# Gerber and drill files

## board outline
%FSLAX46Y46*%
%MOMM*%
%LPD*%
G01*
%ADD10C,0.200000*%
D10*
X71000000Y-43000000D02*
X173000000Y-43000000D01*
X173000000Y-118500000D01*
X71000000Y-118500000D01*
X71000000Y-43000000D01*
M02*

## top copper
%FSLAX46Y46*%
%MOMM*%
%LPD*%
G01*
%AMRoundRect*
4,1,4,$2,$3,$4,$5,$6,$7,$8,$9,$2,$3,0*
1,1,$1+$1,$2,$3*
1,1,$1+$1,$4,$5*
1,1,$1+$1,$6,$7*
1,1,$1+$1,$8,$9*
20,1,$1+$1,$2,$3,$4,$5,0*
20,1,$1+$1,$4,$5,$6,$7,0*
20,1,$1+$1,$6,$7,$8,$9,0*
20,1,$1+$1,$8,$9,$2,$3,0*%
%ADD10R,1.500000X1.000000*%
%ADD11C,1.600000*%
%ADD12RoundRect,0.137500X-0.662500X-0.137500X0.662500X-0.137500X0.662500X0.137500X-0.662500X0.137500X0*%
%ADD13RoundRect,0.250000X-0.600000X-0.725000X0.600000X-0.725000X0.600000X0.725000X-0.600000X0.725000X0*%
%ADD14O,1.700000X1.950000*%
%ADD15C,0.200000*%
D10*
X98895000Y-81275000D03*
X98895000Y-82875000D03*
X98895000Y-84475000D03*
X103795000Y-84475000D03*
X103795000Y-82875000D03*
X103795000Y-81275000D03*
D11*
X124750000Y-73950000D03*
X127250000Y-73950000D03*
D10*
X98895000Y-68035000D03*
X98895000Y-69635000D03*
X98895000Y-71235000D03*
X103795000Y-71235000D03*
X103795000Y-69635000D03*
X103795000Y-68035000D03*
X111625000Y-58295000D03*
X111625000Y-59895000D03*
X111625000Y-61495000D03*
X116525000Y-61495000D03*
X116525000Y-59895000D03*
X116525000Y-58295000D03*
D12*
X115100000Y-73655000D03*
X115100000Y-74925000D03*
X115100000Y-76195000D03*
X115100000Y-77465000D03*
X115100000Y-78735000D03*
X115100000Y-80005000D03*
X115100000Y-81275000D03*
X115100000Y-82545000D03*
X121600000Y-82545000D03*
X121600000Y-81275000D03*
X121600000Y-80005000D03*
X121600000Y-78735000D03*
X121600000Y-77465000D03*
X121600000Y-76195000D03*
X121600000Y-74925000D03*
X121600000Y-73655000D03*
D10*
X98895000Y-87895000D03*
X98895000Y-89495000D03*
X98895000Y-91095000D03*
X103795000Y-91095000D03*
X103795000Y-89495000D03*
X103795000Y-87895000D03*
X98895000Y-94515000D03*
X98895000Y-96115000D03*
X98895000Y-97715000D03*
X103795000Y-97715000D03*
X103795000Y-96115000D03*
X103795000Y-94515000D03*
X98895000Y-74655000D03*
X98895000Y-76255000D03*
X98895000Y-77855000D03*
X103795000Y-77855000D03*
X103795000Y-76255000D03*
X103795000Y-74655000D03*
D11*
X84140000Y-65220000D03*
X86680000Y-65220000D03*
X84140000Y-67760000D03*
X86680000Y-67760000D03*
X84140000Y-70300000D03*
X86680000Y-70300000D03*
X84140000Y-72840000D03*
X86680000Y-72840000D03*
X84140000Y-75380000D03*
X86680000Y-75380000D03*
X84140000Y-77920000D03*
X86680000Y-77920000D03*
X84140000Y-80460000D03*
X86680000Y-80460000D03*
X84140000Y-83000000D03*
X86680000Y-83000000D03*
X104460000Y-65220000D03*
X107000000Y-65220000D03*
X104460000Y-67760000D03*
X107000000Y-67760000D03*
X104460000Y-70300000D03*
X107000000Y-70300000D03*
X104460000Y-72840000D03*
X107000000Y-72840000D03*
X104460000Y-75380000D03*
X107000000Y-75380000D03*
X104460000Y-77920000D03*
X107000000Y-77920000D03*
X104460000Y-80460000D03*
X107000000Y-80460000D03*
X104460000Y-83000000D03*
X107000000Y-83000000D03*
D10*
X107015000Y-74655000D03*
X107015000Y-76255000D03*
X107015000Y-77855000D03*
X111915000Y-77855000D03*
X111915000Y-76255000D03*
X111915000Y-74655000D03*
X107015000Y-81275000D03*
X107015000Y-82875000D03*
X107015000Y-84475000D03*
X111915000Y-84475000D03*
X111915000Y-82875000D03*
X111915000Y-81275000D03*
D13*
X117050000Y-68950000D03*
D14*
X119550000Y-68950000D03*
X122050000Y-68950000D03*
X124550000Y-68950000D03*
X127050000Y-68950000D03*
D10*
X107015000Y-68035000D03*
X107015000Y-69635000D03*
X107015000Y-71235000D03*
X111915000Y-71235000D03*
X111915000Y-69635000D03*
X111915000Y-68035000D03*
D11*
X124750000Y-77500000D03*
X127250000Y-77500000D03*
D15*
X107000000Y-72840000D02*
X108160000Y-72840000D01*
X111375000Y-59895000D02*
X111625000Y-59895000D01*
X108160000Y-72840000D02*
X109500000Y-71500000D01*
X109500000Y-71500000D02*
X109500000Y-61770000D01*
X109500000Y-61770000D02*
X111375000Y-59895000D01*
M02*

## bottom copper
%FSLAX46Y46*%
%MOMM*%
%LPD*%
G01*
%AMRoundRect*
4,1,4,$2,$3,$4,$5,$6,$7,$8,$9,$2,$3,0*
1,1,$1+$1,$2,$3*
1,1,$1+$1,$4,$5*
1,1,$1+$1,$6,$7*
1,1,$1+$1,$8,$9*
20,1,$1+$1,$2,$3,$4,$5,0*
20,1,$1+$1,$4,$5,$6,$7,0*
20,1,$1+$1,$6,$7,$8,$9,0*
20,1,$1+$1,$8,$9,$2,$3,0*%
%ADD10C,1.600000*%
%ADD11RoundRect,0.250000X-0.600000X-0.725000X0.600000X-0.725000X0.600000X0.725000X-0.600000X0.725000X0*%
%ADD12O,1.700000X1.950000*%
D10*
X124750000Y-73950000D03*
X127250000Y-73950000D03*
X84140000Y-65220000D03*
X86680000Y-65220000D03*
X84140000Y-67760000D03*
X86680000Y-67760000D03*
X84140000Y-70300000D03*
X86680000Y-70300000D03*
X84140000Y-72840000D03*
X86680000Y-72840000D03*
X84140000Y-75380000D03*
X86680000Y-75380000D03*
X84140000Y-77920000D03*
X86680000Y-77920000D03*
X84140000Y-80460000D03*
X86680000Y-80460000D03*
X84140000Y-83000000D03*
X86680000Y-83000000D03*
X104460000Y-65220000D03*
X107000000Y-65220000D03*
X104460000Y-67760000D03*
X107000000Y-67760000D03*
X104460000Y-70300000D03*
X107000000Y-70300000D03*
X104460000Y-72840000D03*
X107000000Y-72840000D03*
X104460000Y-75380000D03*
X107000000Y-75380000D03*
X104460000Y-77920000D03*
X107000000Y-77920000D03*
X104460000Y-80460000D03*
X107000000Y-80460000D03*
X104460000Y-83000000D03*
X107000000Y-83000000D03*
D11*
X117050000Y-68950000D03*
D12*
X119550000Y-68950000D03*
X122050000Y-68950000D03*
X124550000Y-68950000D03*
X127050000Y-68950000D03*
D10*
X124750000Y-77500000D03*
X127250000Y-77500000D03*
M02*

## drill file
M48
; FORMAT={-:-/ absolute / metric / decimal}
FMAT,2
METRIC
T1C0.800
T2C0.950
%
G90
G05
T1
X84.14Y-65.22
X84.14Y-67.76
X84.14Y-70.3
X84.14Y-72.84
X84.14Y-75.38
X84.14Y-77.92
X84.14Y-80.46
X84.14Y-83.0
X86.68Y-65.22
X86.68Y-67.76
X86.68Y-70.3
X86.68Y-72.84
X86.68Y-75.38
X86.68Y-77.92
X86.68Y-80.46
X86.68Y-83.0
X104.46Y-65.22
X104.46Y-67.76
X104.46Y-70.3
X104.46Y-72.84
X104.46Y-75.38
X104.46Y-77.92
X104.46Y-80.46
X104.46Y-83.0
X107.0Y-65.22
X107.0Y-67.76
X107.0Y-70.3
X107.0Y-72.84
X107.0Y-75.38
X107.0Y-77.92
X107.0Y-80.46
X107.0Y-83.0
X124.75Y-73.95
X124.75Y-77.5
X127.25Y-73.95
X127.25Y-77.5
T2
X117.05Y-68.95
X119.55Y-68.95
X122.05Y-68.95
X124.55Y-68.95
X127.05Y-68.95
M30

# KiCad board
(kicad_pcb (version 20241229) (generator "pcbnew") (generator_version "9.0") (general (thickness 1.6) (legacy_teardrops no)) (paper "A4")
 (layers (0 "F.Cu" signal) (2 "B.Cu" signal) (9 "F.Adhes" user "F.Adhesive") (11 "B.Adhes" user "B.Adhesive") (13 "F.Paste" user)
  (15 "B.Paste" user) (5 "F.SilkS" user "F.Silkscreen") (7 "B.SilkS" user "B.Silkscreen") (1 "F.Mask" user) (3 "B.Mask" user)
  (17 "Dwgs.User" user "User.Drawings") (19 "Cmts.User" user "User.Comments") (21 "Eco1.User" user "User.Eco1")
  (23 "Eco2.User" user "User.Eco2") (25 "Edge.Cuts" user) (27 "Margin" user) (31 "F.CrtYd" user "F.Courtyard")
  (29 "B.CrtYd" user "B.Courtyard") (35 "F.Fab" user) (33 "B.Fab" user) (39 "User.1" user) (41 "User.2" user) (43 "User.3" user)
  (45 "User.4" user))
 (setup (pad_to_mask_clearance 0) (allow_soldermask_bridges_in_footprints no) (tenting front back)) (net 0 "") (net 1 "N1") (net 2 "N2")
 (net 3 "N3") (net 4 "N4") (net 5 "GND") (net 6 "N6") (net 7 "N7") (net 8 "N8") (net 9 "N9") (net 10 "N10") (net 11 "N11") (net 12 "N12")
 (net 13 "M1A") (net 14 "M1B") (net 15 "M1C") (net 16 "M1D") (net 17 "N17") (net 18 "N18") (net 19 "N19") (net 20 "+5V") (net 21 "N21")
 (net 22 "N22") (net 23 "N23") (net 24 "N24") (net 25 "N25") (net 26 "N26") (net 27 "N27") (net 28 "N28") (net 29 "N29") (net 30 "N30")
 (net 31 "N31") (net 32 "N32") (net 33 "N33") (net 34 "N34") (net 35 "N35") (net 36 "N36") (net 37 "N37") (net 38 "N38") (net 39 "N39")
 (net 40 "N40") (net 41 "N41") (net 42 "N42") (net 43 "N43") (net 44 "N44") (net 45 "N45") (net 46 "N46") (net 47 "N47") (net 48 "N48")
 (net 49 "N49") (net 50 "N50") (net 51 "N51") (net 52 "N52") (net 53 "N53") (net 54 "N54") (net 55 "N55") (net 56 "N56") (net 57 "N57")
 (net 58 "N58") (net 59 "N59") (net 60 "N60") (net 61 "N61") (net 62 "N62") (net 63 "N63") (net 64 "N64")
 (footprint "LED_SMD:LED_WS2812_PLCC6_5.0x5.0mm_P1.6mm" (layer "F.Cu") (at 101.345 82.875)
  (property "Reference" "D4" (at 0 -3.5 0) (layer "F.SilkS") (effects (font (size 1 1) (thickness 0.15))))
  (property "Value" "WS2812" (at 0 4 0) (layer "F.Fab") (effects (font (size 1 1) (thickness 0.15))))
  (pad "1" smd rect (at -2.45 -1.6) (size 1.5 1) (layers "F.Cu" "F.Mask" "F.Paste") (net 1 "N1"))
  (pad "2" smd rect (at -2.45 0) (size 1.5 1) (layers "F.Cu" "F.Mask" "F.Paste") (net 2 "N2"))
  (pad "3" smd rect (at -2.45 1.6) (size 1.5 1) (layers "F.Cu" "F.Mask" "F.Paste") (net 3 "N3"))
  (pad "4" smd rect (at 2.45 1.6) (size 1.5 1) (layers "F.Cu" "F.Mask" "F.Paste") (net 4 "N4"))
  (pad "5" smd rect (at 2.45 0) (size 1.5 1) (layers "F.Cu" "F.Mask" "F.Paste") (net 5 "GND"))
  (pad "6" smd rect (at 2.45 -1.6) (size 1.5 1) (layers "F.Cu" "F.Mask" "F.Paste") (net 5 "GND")))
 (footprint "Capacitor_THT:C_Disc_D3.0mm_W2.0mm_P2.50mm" (layer "F.Cu") (at 124.75 73.95)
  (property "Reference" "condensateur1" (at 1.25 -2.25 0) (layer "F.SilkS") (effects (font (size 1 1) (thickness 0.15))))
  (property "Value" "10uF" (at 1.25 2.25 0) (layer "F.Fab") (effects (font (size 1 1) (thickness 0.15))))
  (pad "1" thru_hole circle (at 0 0) (size 1.6 1.6) (drill 0.8) (layers "*.Cu" "*.Mask") (remove_unused_layers no) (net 5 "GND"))
  (pad "2" thru_hole circle (at 2.5 0) (size 1.6 1.6) (drill 0.8) (layers "*.Cu" "*.Mask") (remove_unused_layers no) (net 5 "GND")))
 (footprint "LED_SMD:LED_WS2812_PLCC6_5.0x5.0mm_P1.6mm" (layer "F.Cu") (at 101.345 69.635)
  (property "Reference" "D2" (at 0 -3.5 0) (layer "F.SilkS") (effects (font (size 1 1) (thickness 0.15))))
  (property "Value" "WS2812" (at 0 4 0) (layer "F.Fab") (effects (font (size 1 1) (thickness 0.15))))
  (pad "1" smd rect (at -2.45 -1.6) (size 1.5 1) (layers "F.Cu" "F.Mask" "F.Paste") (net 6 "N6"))
  (pad "2" smd rect (at -2.45 0) (size 1.5 1) (layers "F.Cu" "F.Mask" "F.Paste") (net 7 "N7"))
  (pad "3" smd rect (at -2.45 1.6) (size 1.5 1) (layers "F.Cu" "F.Mask" "F.Paste") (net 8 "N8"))
  (pad "4" smd rect (at 2.45 1.6) (size 1.5 1) (layers "F.Cu" "F.Mask" "F.Paste") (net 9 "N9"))
  (pad "5" smd rect (at 2.45 0) (size 1.5 1) (layers "F.Cu" "F.Mask" "F.Paste") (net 5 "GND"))
  (pad "6" smd rect (at 2.45 -1.6) (size 1.5 1) (layers "F.Cu" "F.Mask" "F.Paste") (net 5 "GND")))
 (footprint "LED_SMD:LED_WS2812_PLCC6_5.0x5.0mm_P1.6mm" (layer "F.Cu") (at 114.075 59.895)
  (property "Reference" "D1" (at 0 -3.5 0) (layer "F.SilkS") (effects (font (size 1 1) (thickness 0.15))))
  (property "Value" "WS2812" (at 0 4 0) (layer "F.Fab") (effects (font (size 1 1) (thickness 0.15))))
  (pad "1" smd rect (at -2.45 -1.6) (size 1.5 1) (layers "F.Cu" "F.Mask" "F.Paste") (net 7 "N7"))
  (pad "2" smd rect (at -2.45 0) (size 1.5 1) (layers "F.Cu" "F.Mask" "F.Paste") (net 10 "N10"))
  (pad "3" smd rect (at -2.45 1.6) (size 1.5 1) (layers "F.Cu" "F.Mask" "F.Paste") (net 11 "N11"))
  (pad "4" smd rect (at 2.45 1.6) (size 1.5 1) (layers "F.Cu" "F.Mask" "F.Paste") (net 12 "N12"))
  (pad "5" smd rect (at 2.45 0) (size 1.5 1) (layers "F.Cu" "F.Mask" "F.Paste") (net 5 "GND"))
  (pad "6" smd rect (at 2.45 -1.6) (size 1.5 1) (layers "F.Cu" "F.Mask" "F.Paste") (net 5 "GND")))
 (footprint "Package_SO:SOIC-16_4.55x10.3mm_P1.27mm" (layer "F.Cu") (at 118.35 78.1)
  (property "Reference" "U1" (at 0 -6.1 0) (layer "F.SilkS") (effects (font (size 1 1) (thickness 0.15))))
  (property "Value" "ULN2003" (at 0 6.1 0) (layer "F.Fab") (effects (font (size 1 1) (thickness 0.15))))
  (pad "1" smd roundrect (at -3.25 -4.445) (size 1.6 0.55) (layers "F.Cu" "F.Mask" "F.Paste") (roundrect_rratio 0.25) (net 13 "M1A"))
  (pad "2" smd roundrect (at -3.25 -3.175) (size 1.6 0.55) (layers "F.Cu" "F.Mask" "F.Paste") (roundrect_rratio 0.25) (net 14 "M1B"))
  (pad "3" smd roundrect (at -3.25 -1.905) (size 1.6 0.55) (layers "F.Cu" "F.Mask" "F.Paste") (roundrect_rratio 0.25) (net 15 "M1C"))
  (pad "4" smd roundrect (at -3.25 -0.635) (size 1.6 0.55) (layers "F.Cu" "F.Mask" "F.Paste") (roundrect_rratio 0.25) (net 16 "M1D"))
  (pad "5" smd roundrect (at -3.25 0.635) (size 1.6 0.55) (layers "F.Cu" "F.Mask" "F.Paste") (roundrect_rratio 0.25) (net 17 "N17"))
  (pad "6" smd roundrect (at -3.25 1.905) (size 1.6 0.55) (layers "F.Cu" "F.Mask" "F.Paste") (roundrect_rratio 0.25) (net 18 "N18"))
  (pad "7" smd roundrect (at -3.25 3.175) (size 1.6 0.55) (layers "F.Cu" "F.Mask" "F.Paste") (roundrect_rratio 0.25) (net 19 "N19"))
  (pad "8" smd roundrect (at -3.25 4.445) (size 1.6 0.55) (layers "F.Cu" "F.Mask" "F.Paste") (roundrect_rratio 0.25) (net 5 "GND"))
  (pad "9" smd roundrect (at 3.25 4.445) (size 1.6 0.55) (layers "F.Cu" "F.Mask" "F.Paste") (roundrect_rratio 0.25) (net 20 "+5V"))
  (pad "10" smd roundrect (at 3.25 3.175) (size 1.6 0.55) (layers "F.Cu" "F.Mask" "F.Paste") (roundrect_rratio 0.25) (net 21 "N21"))
  (pad "11" smd roundrect (at 3.25 1.905) (size 1.6 0.55) (layers "F.Cu" "F.Mask" "F.Paste") (roundrect_rratio 0.25) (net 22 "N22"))
  (pad "12" smd roundrect (at 3.25 0.635) (size 1.6 0.55) (layers "F.Cu" "F.Mask" "F.Paste") (roundrect_rratio 0.25) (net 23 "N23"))
  (pad "13" smd roundrect (at 3.25 -0.635) (size 1.6 0.55) (layers "F.Cu" "F.Mask" "F.Paste") (roundrect_rratio 0.25) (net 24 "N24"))
  (pad "14" smd roundrect (at 3.25 -1.905) (size 1.6 0.55) (layers "F.Cu" "F.Mask" "F.Paste") (roundrect_rratio 0.25) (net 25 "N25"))
  (pad "15" smd roundrect (at 3.25 -3.175) (size 1.6 0.55) (layers "F.Cu" "F.Mask" "F.Paste") (roundrect_rratio 0.25) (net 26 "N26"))
  (pad "16" smd roundrect (at 3.25 -4.445) (size 1.6 0.55) (layers "F.Cu" "F.Mask" "F.Paste") (roundrect_rratio 0.25) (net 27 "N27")))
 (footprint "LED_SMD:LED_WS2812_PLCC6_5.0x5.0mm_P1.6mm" (layer "F.Cu") (at 101.345 89.495)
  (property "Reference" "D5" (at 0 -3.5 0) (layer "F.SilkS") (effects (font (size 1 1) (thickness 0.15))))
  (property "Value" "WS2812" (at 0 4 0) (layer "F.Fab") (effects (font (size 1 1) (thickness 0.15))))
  (pad "1" smd rect (at -2.45 -1.6) (size 1.5 1) (layers "F.Cu" "F.Mask" "F.Paste") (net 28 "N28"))
  (pad "2" smd rect (at -2.45 0) (size 1.5 1) (layers "F.Cu" "F.Mask" "F.Paste") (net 1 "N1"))
  (pad "3" smd rect (at -2.45 1.6) (size 1.5 1) (layers "F.Cu" "F.Mask" "F.Paste") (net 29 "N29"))
  (pad "4" smd rect (at 2.45 1.6) (size 1.5 1) (layers "F.Cu" "F.Mask" "F.Paste") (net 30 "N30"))
  (pad "5" smd rect (at 2.45 0) (size 1.5 1) (layers "F.Cu" "F.Mask" "F.Paste") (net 5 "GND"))
  (pad "6" smd rect (at 2.45 -1.6) (size 1.5 1) (layers "F.Cu" "F.Mask" "F.Paste") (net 5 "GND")))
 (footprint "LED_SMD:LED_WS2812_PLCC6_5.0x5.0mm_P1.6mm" (layer "F.Cu") (at 101.345 96.115)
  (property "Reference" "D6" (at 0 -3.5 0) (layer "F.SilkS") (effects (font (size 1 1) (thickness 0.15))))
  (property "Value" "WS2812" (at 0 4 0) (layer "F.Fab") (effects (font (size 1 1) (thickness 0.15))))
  (pad "1" smd rect (at -2.45 -1.6) (size 1.5 1) (layers "F.Cu" "F.Mask" "F.Paste") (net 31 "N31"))
  (pad "2" smd rect (at -2.45 0) (size 1.5 1) (layers "F.Cu" "F.Mask" "F.Paste") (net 28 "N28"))
  (pad "3" smd rect (at -2.45 1.6) (size 1.5 1) (layers "F.Cu" "F.Mask" "F.Paste") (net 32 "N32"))
  (pad "4" smd rect (at 2.45 1.6) (size 1.5 1) (layers "F.Cu" "F.Mask" "F.Paste") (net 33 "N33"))
  (pad "5" smd rect (at 2.45 0) (size 1.5 1) (layers "F.Cu" "F.Mask" "F.Paste") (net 5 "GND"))
  (pad "6" smd rect (at 2.45 -1.6) (size 1.5 1) (layers "F.Cu" "F.Mask" "F.Paste") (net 5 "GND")))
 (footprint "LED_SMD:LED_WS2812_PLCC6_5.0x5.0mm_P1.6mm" (layer "F.Cu") (at 101.345 76.255)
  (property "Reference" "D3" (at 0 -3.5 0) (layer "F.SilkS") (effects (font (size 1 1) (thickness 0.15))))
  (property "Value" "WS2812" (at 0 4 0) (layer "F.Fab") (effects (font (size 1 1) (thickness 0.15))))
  (pad "1" smd rect (at -2.45 -1.6) (size 1.5 1) (layers "F.Cu" "F.Mask" "F.Paste") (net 2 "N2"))
  (pad "2" smd rect (at -2.45 0) (size 1.5 1) (layers "F.Cu" "F.Mask" "F.Paste") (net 6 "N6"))
  (pad "3" smd rect (at -2.45 1.6) (size 1.5 1) (layers "F.Cu" "F.Mask" "F.Paste") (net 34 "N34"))
  (pad "4" smd rect (at 2.45 1.6) (size 1.5 1) (layers "F.Cu" "F.Mask" "F.Paste") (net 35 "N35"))
  (pad "5" smd rect (at 2.45 0) (size 1.5 1) (layers "F.Cu" "F.Mask" "F.Paste") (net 5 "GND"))
  (pad "6" smd rect (at 2.45 -1.6) (size 1.5 1) (layers "F.Cu" "F.Mask" "F.Paste") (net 5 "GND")))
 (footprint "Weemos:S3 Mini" (layer "F.Cu") (at 95.57 74.11)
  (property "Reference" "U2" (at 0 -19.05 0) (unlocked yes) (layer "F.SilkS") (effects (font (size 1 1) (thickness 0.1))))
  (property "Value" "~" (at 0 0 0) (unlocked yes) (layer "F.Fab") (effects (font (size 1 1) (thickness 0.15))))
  (pad "1" thru_hole circle (at -11.43 -8.89) (size 1.6 1.6) (drill 0.8) (layers "*.Cu" "*.Mask") (remove_unused_layers no) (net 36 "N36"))
  (pad "2" thru_hole circle (at -8.89 -8.89) (size 1.6 1.6) (drill 0.8) (layers "*.Cu" "*.Mask") (remove_unused_layers no) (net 13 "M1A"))
  (pad "3" thru_hole circle (at -11.43 -6.35) (size 1.6 1.6) (drill 0.8) (layers "*.Cu" "*.Mask") (remove_unused_layers no) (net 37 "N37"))
  (pad "4" thru_hole circle (at -8.89 -6.35) (size 1.6 1.6) (drill 0.8) (layers "*.Cu" "*.Mask") (remove_unused_layers no) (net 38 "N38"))
  (pad "5" thru_hole circle (at -11.43 -3.81) (size 1.6 1.6) (drill 0.8) (layers "*.Cu" "*.Mask") (remove_unused_layers no) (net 14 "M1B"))
  (pad "6" thru_hole circle (at -8.89 -3.81) (size 1.6 1.6) (drill 0.8) (layers "*.Cu" "*.Mask") (remove_unused_layers no) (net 15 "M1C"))
  (pad "7" thru_hole circle (at -11.43 -1.27) (size 1.6 1.6) (drill 0.8) (layers "*.Cu" "*.Mask") (remove_unused_layers no) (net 16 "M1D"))
  (pad "8" thru_hole circle (at -8.89 -1.27) (size 1.6 1.6) (drill 0.8) (layers "*.Cu" "*.Mask") (remove_unused_layers no) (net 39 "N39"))
  (pad "9" thru_hole circle (at -11.43 1.27) (size 1.6 1.6) (drill 0.8) (layers "*.Cu" "*.Mask") (remove_unused_layers no) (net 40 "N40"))
  (pad "10" thru_hole circle (at -8.89 1.27) (size 1.6 1.6) (drill 0.8) (layers "*.Cu" "*.Mask") (remove_unused_layers no) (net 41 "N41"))
  (pad "11" thru_hole circle (at -11.43 3.81) (size 1.6 1.6) (drill 0.8) (layers "*.Cu" "*.Mask") (remove_unused_layers no) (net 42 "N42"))
  (pad "12" thru_hole circle (at -8.89 3.81) (size 1.6 1.6) (drill 0.8) (layers "*.Cu" "*.Mask") (remove_unused_layers no) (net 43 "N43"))
  (pad "13" thru_hole circle (at -11.43 6.35) (size 1.6 1.6) (drill 0.8) (layers "*.Cu" "*.Mask") (remove_unused_layers no) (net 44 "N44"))
  (pad "14" thru_hole circle (at -8.89 6.35) (size 1.6 1.6) (drill 0.8) (layers "*.Cu" "*.Mask") (remove_unused_layers no) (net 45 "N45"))
  (pad "15" thru_hole circle (at -11.43 8.89) (size 1.6 1.6) (drill 0.8) (layers "*.Cu" "*.Mask") (remove_unused_layers no) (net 5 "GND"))
  (pad "16" thru_hole circle (at -8.89 8.89) (size 1.6 1.6) (drill 0.8) (layers "*.Cu" "*.Mask") (remove_unused_layers no) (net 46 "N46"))
  (pad "17" thru_hole circle (at 8.89 -8.89) (size 1.6 1.6) (drill 0.8) (layers "*.Cu" "*.Mask") (remove_unused_layers no) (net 10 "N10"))
  (pad "18" thru_hole circle (at 11.43 -8.89) (size 1.6 1.6) (drill 0.8) (layers "*.Cu" "*.Mask") (remove_unused_layers no) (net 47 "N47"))
  (pad "19" thru_hole circle (at 8.89 -6.35) (size 1.6 1.6) (drill 0.8) (layers "*.Cu" "*.Mask") (remove_unused_layers no) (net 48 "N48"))
  (pad "20" thru_hole circle (at 11.43 -6.35) (size 1.6 1.6) (drill 0.8) (layers "*.Cu" "*.Mask") (remove_unused_layers no) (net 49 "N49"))
  (pad "21" thru_hole circle (at 8.89 -3.81) (size 1.6 1.6) (drill 0.8) (layers "*.Cu" "*.Mask") (remove_unused_layers no) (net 5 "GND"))
  (pad "22" thru_hole circle (at 11.43 -3.81) (size 1.6 1.6) (drill 0.8) (layers "*.Cu" "*.Mask") (remove_unused_layers no) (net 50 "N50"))
  (pad "23" thru_hole circle (at 8.89 -1.27) (size 1.6 1.6) (drill 0.8) (layers "*.Cu" "*.Mask") (remove_unused_layers no) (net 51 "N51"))
  (pad "24" thru_hole circle (at 11.43 -1.27) (size 1.6 1.6) (drill 0.8) (layers "*.Cu" "*.Mask") (remove_unused_layers no) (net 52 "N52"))
  (pad "25" thru_hole circle (at 8.89 1.27) (size 1.6 1.6) (drill 0.8) (layers "*.Cu" "*.Mask") (remove_unused_layers no) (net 5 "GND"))
  (pad "26" thru_hole circle (at 11.43 1.27) (size 1.6 1.6) (drill 0.8) (layers "*.Cu" "*.Mask") (remove_unused_layers no) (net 5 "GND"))
  (pad "27" thru_hole circle (at 8.89 3.81) (size 1.6 1.6) (drill 0.8) (layers "*.Cu" "*.Mask") (remove_unused_layers no) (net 5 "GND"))
  (pad "28" thru_hole circle (at 11.43 3.81) (size 1.6 1.6) (drill 0.8) (layers "*.Cu" "*.Mask") (remove_unused_layers no) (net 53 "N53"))
  (pad "29" thru_hole circle (at 8.89 6.35) (size 1.6 1.6) (drill 0.8) (layers "*.Cu" "*.Mask") (remove_unused_layers no) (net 5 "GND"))
  (pad "30" thru_hole circle (at 11.43 6.35) (size 1.6 1.6) (drill 0.8) (layers "*.Cu" "*.Mask") (remove_unused_layers no) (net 5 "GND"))
  (pad "31" thru_hole circle (at 8.89 8.89) (size 1.6 1.6) (drill 0.8) (layers "*.Cu" "*.Mask") (remove_unused_layers no) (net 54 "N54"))
  (pad "32" thru_hole circle (at 11.43 8.89) (size 1.6 1.6) (drill 0.8) (layers "*.Cu" "*.Mask") (remove_unused_layers no) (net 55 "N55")))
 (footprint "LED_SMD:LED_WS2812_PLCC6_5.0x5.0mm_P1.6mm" (layer "F.Cu") (at 109.465 76.255)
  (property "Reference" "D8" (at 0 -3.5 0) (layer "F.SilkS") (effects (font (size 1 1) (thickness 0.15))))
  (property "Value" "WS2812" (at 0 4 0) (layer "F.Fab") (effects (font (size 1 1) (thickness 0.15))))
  (pad "1" smd rect (at -2.45 -1.6) (size 1.5 1) (layers "F.Cu" "F.Mask" "F.Paste") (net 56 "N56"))
  (pad "2" smd rect (at -2.45 0) (size 1.5 1) (layers "F.Cu" "F.Mask" "F.Paste") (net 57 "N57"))
  (pad "3" smd rect (at -2.45 1.6) (size 1.5 1) (layers "F.Cu" "F.Mask" "F.Paste") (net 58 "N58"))
  (pad "4" smd rect (at 2.45 1.6) (size 1.5 1) (layers "F.Cu" "F.Mask" "F.Paste") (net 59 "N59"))
  (pad "5" smd rect (at 2.45 0) (size 1.5 1) (layers "F.Cu" "F.Mask" "F.Paste") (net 5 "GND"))
  (pad "6" smd rect (at 2.45 -1.6) (size 1.5 1) (layers "F.Cu" "F.Mask" "F.Paste") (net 5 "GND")))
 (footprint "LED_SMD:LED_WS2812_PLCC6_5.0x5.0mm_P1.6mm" (layer "F.Cu") (at 109.465 82.875)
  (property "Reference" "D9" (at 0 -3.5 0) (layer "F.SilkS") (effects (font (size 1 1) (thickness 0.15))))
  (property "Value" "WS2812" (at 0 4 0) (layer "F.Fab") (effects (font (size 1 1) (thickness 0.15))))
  (pad "1" smd rect (at -2.45 -1.6) (size 1.5 1) (layers "F.Cu" "F.Mask" "F.Paste") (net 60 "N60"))
  (pad "2" smd rect (at -2.45 0) (size 1.5 1) (layers "F.Cu" "F.Mask" "F.Paste") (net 56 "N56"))
  (pad "3" smd rect (at -2.45 1.6) (size 1.5 1) (layers "F.Cu" "F.Mask" "F.Paste") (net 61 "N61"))
  (pad "4" smd rect (at 2.45 1.6) (size 1.5 1) (layers "F.Cu" "F.Mask" "F.Paste") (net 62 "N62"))
  (pad "5" smd rect (at 2.45 0) (size 1.5 1) (layers "F.Cu" "F.Mask" "F.Paste") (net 5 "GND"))
  (pad "6" smd rect (at 2.45 -1.6) (size 1.5 1) (layers "F.Cu" "F.Mask" "F.Paste") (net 5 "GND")))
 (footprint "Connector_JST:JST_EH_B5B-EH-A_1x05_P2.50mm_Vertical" (layer "F.Cu") (at 117.05 68.95)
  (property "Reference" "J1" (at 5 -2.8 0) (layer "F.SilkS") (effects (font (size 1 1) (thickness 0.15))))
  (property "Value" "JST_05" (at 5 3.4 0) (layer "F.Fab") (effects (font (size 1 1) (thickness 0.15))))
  (pad "1" thru_hole roundrect (at 0 0) (size 1.7 1.95) (drill 0.95) (layers "*.Cu" "*.Mask") (remove_unused_layers no)
   (roundrect_rratio 0.147059) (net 20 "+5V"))
  (pad "2" thru_hole oval (at 2.5 0) (size 1.7 1.95) (drill 0.95) (layers "*.Cu" "*.Mask") (remove_unused_layers no) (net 27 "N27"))
  (pad "3" thru_hole oval (at 5 0) (size 1.7 1.95) (drill 0.95) (layers "*.Cu" "*.Mask") (remove_unused_layers no) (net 26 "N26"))
  (pad "4" thru_hole oval (at 7.5 0) (size 1.7 1.95) (drill 0.95) (layers "*.Cu" "*.Mask") (remove_unused_layers no) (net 25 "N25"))
  (pad "5" thru_hole oval (at 10 0) (size 1.7 1.95) (drill 0.95) (layers "*.Cu" "*.Mask") (remove_unused_layers no) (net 24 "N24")))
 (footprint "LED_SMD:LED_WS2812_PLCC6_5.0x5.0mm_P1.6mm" (layer "F.Cu") (at 109.465 69.635)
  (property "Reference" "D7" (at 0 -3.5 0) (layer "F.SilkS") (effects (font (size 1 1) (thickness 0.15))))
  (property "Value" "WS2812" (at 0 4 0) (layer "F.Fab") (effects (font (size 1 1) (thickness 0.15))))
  (pad "1" smd rect (at -2.45 -1.6) (size 1.5 1) (layers "F.Cu" "F.Mask" "F.Paste") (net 57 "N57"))
  (pad "2" smd rect (at -2.45 0) (size 1.5 1) (layers "F.Cu" "F.Mask" "F.Paste") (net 31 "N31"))
  (pad "3" smd rect (at -2.45 1.6) (size 1.5 1) (layers "F.Cu" "F.Mask" "F.Paste") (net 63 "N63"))
  (pad "4" smd rect (at 2.45 1.6) (size 1.5 1) (layers "F.Cu" "F.Mask" "F.Paste") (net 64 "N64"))
  (pad "5" smd rect (at 2.45 0) (size 1.5 1) (layers "F.Cu" "F.Mask" "F.Paste") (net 5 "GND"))
  (pad "6" smd rect (at 2.45 -1.6) (size 1.5 1) (layers "F.Cu" "F.Mask" "F.Paste") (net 5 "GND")))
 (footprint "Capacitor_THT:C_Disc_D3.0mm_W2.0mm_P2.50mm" (layer "F.Cu") (at 124.75 77.5)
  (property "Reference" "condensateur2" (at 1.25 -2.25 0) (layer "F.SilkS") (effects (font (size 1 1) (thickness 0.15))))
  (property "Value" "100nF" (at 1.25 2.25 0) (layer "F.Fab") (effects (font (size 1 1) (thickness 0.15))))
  (pad "1" thru_hole circle (at 0 0) (size 1.6 1.6) (drill 0.8) (layers "*.Cu" "*.Mask") (remove_unused_layers no) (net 5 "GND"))
  (pad "2" thru_hole circle (at 2.5 0) (size 1.6 1.6) (drill 0.8) (layers "*.Cu" "*.Mask") (remove_unused_layers no) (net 5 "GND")))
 (gr_rect (start 71 43) (end 173 118.5) (stroke (width 0.2) (type solid)) (fill no) (layer "Edge.Cuts"))
 (segment (start 107 72.84) (end 108.16 72.84) (width 0.2) (layer "F.Cu") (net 10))
 (segment (start 111.375 59.895) (end 111.625 59.895) (width 0.2) (layer "F.Cu") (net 10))
 (segment (start 108.16 72.84) (end 109.5 71.5) (width 0.2) (layer "F.Cu") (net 10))
 (segment (start 109.5 71.5) (end 109.5 61.77) (width 0.2) (layer "F.Cu") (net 10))
 (segment (start 109.5 61.77) (end 111.375 59.895) (width 0.2) (layer "F.Cu") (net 10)))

